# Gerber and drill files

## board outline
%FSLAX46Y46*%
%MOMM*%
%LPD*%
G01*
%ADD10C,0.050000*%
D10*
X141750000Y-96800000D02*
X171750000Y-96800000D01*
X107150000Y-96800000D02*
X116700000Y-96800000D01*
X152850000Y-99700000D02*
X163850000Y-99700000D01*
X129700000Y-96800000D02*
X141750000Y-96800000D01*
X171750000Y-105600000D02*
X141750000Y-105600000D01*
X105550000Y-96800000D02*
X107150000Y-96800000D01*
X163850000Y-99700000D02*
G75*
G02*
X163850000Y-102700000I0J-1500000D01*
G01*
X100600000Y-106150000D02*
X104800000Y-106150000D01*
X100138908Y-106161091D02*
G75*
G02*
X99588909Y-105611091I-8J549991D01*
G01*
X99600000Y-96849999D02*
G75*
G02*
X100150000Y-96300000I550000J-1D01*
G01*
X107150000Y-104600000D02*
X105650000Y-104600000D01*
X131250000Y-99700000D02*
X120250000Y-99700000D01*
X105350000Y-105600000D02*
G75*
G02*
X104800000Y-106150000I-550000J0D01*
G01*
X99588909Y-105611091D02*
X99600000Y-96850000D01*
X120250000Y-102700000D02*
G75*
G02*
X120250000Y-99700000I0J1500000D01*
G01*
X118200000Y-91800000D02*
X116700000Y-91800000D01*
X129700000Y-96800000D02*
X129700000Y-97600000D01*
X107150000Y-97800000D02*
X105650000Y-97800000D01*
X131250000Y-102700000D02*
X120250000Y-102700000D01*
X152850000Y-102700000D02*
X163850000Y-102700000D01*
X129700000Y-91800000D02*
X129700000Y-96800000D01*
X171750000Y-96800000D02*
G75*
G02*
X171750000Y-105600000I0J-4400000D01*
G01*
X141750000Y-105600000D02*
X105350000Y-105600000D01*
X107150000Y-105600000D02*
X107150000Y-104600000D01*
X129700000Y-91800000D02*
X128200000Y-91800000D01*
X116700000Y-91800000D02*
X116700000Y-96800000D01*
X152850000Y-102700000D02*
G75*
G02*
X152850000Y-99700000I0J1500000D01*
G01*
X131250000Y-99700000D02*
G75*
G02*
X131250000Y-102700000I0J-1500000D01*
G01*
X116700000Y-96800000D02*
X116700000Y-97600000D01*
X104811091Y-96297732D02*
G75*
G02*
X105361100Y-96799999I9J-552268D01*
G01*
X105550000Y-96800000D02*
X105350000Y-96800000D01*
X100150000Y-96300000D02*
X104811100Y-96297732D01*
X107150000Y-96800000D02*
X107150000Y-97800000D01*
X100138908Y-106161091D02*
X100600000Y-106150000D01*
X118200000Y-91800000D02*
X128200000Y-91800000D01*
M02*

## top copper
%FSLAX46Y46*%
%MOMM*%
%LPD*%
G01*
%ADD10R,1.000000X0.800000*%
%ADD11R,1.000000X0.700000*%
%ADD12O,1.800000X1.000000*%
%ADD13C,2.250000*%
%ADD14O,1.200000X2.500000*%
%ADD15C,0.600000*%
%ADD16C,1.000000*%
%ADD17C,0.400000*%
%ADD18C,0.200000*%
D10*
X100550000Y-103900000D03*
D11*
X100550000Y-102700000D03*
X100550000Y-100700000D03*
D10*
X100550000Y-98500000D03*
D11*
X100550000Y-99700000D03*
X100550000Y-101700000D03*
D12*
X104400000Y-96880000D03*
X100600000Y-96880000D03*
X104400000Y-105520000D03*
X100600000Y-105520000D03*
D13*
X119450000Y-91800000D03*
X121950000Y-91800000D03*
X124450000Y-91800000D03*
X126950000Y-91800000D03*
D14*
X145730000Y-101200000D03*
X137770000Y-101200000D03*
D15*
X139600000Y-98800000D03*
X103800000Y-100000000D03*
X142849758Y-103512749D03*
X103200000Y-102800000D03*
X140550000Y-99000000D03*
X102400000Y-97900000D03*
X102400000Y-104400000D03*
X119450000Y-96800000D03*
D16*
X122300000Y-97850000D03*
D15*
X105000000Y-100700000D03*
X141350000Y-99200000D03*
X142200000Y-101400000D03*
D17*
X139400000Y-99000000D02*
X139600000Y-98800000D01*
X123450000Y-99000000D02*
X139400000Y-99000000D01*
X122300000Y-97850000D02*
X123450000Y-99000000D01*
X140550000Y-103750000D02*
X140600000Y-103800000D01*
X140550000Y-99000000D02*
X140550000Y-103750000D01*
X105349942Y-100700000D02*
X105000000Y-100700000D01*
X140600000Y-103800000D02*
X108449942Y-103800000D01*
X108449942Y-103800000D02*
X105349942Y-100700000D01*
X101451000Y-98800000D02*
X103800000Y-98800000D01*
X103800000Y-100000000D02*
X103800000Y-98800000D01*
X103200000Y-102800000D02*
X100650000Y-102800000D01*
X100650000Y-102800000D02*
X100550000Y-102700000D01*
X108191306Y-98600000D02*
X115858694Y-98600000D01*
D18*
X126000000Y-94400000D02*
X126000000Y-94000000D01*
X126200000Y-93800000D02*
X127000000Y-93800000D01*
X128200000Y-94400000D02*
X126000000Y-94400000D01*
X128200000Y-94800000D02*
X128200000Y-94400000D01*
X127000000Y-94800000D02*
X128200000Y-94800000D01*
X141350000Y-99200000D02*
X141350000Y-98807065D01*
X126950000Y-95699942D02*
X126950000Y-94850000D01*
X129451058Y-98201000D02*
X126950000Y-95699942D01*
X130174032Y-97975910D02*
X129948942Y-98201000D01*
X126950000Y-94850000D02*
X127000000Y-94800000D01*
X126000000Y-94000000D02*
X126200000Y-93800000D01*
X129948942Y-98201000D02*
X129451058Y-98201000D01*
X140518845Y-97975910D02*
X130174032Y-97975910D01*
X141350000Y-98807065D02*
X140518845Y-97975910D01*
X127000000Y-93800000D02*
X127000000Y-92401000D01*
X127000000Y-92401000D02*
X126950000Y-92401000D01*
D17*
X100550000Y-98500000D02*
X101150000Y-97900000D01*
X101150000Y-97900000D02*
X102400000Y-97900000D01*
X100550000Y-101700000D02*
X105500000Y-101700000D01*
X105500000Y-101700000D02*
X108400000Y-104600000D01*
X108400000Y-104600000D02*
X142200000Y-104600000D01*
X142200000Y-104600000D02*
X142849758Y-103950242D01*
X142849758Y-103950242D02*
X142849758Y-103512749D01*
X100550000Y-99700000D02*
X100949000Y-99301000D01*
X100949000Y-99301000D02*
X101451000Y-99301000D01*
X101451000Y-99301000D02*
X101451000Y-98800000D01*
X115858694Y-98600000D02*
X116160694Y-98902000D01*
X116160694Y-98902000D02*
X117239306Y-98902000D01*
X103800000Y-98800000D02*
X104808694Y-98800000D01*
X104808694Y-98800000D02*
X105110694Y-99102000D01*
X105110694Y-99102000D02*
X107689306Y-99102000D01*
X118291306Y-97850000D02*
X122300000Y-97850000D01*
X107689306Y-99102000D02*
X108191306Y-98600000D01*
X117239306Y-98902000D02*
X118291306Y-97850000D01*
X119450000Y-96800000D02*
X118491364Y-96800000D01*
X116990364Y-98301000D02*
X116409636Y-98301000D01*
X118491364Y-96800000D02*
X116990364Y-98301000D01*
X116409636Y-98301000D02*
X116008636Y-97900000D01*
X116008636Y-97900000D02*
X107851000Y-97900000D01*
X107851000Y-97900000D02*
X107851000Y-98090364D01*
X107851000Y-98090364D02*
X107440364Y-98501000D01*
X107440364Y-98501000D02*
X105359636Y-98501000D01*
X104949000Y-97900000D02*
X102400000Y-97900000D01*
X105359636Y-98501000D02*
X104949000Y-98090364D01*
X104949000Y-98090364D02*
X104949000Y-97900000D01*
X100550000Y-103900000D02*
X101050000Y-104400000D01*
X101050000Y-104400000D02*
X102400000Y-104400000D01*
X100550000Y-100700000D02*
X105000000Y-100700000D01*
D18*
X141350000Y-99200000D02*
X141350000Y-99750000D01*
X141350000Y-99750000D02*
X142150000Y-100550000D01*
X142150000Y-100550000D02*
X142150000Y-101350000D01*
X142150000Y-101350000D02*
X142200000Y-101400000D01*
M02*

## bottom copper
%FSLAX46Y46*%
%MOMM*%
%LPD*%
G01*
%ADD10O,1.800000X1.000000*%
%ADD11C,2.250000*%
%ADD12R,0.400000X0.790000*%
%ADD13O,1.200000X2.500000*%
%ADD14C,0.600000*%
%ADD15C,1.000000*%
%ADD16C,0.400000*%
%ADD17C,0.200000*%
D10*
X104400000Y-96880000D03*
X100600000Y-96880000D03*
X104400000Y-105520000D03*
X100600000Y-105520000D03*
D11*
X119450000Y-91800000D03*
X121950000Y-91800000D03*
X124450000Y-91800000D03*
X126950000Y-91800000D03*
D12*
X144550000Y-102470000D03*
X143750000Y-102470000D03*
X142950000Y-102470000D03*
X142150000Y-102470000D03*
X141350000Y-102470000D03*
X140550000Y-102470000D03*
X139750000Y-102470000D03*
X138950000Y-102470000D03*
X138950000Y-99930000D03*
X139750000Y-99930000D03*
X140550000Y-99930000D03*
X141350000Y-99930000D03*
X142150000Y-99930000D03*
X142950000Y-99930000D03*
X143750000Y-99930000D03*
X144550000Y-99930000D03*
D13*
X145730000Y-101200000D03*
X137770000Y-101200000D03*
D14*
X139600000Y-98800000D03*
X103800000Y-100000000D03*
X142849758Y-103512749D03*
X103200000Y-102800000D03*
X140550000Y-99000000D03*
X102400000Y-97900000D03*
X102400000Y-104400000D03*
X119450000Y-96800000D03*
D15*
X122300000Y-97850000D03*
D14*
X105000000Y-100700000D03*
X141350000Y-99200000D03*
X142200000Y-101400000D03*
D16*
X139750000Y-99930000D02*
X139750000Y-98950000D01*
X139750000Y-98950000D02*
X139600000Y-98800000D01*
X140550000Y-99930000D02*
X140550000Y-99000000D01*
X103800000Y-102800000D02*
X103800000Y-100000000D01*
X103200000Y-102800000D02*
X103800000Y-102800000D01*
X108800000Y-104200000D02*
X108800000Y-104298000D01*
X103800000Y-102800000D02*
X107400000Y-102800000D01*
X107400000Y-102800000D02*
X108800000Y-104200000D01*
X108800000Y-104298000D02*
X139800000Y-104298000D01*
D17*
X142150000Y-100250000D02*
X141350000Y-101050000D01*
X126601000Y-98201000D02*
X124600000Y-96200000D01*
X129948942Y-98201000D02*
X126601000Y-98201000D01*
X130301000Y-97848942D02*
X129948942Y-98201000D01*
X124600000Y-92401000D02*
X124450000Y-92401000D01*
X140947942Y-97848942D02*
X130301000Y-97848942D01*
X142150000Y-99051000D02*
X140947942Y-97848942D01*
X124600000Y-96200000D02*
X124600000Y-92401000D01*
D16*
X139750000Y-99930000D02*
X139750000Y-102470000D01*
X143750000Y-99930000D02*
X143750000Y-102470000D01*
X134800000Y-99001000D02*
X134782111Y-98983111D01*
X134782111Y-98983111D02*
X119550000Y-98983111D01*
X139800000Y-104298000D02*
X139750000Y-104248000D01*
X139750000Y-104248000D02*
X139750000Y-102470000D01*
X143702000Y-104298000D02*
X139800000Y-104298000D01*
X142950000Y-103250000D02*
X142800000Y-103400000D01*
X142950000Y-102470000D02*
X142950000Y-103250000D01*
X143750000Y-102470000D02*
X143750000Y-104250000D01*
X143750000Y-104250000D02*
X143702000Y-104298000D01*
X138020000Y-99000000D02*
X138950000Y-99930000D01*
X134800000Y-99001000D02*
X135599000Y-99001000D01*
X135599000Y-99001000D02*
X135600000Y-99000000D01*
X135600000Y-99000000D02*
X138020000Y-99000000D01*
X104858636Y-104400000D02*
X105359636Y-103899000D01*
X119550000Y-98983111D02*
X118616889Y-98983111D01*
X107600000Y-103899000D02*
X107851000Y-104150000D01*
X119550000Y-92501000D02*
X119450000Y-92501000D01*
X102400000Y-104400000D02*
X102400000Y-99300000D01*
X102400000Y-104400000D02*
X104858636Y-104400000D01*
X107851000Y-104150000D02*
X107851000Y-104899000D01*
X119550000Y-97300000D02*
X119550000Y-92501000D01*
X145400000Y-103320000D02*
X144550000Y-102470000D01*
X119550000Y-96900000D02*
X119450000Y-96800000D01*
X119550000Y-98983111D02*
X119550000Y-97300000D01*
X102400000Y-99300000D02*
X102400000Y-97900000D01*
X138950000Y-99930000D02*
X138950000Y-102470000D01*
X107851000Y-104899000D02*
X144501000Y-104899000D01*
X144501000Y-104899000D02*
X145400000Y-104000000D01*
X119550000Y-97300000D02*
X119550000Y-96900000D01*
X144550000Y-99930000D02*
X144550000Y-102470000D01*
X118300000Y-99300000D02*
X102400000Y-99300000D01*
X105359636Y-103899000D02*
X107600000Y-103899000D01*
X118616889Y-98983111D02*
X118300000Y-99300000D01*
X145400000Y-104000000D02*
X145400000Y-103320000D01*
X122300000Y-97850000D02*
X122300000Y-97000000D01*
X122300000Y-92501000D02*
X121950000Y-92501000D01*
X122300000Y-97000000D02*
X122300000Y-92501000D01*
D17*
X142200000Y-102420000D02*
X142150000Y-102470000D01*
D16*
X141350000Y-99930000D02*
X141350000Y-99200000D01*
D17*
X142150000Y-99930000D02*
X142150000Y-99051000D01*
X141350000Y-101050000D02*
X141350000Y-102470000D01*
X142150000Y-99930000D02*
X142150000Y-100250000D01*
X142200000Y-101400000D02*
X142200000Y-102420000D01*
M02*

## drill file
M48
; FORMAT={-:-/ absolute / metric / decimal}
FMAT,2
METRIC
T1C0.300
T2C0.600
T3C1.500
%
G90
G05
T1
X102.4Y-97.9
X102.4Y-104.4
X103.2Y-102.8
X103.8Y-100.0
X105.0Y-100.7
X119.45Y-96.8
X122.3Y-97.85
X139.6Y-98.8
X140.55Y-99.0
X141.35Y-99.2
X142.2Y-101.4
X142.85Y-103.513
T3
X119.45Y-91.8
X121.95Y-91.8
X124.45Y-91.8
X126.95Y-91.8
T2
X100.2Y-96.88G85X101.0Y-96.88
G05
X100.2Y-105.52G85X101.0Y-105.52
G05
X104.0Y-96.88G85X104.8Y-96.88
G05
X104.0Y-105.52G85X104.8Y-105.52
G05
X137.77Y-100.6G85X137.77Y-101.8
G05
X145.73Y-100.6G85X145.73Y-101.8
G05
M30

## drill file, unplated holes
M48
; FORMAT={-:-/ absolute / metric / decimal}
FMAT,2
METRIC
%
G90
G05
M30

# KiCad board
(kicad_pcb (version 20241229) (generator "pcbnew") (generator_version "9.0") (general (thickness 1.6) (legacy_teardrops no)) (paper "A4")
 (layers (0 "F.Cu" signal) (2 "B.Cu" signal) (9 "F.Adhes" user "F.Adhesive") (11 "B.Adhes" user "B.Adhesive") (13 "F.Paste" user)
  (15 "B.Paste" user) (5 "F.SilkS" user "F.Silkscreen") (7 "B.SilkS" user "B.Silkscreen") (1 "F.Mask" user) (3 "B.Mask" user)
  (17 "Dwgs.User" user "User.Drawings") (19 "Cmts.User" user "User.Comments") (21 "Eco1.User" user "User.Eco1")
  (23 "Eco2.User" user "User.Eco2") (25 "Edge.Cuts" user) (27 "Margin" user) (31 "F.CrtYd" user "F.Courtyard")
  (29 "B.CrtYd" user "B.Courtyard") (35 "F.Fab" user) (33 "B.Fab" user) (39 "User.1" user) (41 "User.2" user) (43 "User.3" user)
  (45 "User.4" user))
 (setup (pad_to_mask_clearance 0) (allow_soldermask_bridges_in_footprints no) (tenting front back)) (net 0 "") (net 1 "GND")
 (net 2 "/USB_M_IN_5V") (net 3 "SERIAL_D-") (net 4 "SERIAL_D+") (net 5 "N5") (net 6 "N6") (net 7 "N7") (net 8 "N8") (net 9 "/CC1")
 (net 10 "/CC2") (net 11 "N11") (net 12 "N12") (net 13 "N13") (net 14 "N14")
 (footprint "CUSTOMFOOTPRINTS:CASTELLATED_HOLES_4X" (layer "F.Cu") (at 123.2 91.8)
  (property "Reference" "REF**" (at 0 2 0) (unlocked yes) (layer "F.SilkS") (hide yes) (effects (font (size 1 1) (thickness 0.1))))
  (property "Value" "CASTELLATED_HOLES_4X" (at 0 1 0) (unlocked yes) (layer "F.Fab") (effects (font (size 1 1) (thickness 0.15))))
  (fp_line (start -5 0) (end 5 0) (stroke (width 0.05) (type default)) (layer "Edge.Cuts"))
  (pad "1" thru_hole circle (at -3.75 0) (size 2.25 2.25) (drill 1.5) (layers "*.Cu" "*.Mask") (remove_unused_layers no) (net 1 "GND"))
  (pad "2" thru_hole circle (at -1.25 0) (size 2.25 2.25) (drill 1.5) (layers "*.Cu" "*.Mask") (remove_unused_layers no)
   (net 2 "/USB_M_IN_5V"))
  (pad "3" thru_hole circle (at 1.25 0) (size 2.25 2.25) (drill 1.5) (layers "*.Cu" "*.Mask") (remove_unused_layers no) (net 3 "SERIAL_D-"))
  (pad "4" thru_hole circle (at 3.75 0) (size 2.25 2.25) (drill 1.5) (layers "*.Cu" "*.Mask") (remove_unused_layers no) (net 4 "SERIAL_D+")))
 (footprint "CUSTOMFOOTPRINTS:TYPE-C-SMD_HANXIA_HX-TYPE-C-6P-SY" (layer "F.Cu") (at 102.475 101.2 90)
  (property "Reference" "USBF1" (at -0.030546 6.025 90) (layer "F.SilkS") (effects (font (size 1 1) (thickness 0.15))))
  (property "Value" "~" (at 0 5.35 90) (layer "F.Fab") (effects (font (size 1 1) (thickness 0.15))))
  (pad "7" thru_hole oval (at -4.32 -1.875 90) (size 1 1.8) (drill oval 0.6 1.4) (layers "*.Cu" "*.Mask") (remove_unused_layers no)
   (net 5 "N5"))
  (pad "7" thru_hole oval (at -4.32 1.925 90) (size 1 1.8) (drill oval 0.6 1.4) (layers "*.Cu" "*.Mask") (remove_unused_layers no)
   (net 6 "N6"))
  (pad "7" thru_hole oval (at 4.32 -1.875 90) (size 1 1.8) (drill oval 0.6 1.4) (layers "*.Cu" "*.Mask") (remove_unused_layers no)
   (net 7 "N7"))
  (pad "7" thru_hole oval (at 4.32 1.925 90) (size 1 1.8) (drill oval 0.6 1.4) (layers "*.Cu" "*.Mask") (remove_unused_layers no)
   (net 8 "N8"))
  (pad "A5" smd rect (at -0.5 -1.925 90) (size 0.7 1) (layers "F.Cu" "F.Mask" "F.Paste") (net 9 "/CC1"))
  (pad "A9" smd rect (at 1.5 -1.925 90) (size 0.7 1) (layers "F.Cu" "F.Mask" "F.Paste") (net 2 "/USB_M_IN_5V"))
  (pad "A12" smd rect (at 2.7 -1.925 90) (size 0.8 1) (layers "F.Cu" "F.Mask" "F.Paste") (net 1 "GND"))
  (pad "B5" smd rect (at 0.5 -1.925 90) (size 0.7 1) (layers "F.Cu" "F.Mask" "F.Paste") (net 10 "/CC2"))
  (pad "B9" smd rect (at -1.5 -1.925 90) (size 0.7 1) (layers "F.Cu" "F.Mask" "F.Paste") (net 2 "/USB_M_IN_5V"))
  (pad "B12" smd rect (at -2.7 -1.925 90) (size 0.8 1) (layers "F.Cu" "F.Mask" "F.Paste") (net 1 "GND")))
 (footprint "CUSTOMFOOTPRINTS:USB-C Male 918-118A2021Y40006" (layer "B.Cu") (at 141.75 101.2)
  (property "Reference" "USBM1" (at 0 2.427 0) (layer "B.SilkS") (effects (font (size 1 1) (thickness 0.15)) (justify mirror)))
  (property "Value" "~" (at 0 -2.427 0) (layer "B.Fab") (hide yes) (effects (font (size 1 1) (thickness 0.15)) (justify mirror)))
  (pad "1" smd rect (at 2.8 1.27) (size 0.4 0.79) (layers "B.Cu" "B.Mask" "B.Paste") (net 1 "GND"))
  (pad "2" smd rect (at 2 1.27) (size 0.4 0.79) (layers "B.Cu" "B.Mask" "B.Paste") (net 2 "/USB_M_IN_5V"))
  (pad "3" smd rect (at 1.2 1.27) (size 0.4 0.79) (layers "B.Cu" "B.Mask" "B.Paste") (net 9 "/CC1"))
  (pad "4" smd rect (at 0.4 1.27) (size 0.4 0.79) (layers "B.Cu" "B.Mask" "B.Paste") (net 4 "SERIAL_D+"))
  (pad "5" smd rect (at -0.4 1.27) (size 0.4 0.79) (layers "B.Cu" "B.Mask" "B.Paste") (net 3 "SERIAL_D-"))
  (pad "6" smd rect (at -1.2 1.27) (size 0.4 0.79) (layers "B.Cu" "B.Mask" "B.Paste") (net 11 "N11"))
  (pad "7" smd rect (at -2 1.27) (size 0.4 0.79) (layers "B.Cu" "B.Mask" "B.Paste") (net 2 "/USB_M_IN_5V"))
  (pad "8" smd rect (at -2.8 1.27) (size 0.4 0.79) (layers "B.Cu" "B.Mask" "B.Paste") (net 1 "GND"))
  (pad "9" smd rect (at -2.8 -1.27) (size 0.4 0.79) (layers "B.Cu" "B.Mask" "B.Paste") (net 1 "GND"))
  (pad "10" smd rect (at -2 -1.27) (size 0.4 0.79) (layers "B.Cu" "B.Mask" "B.Paste") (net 2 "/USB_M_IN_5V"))
  (pad "11" smd rect (at -1.2 -1.27) (size 0.4 0.79) (layers "B.Cu" "B.Mask" "B.Paste") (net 10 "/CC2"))
  (pad "12" smd rect (at -0.4 -1.27) (size 0.4 0.79) (layers "B.Cu" "B.Mask" "B.Paste") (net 4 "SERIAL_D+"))
  (pad "13" smd rect (at 0.4 -1.27) (size 0.4 0.79) (layers "B.Cu" "B.Mask" "B.Paste") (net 3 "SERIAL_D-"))
  (pad "14" smd rect (at 1.2 -1.27) (size 0.4 0.79) (layers "B.Cu" "B.Mask" "B.Paste") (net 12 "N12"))
  (pad "15" smd rect (at 2 -1.27) (size 0.4 0.79) (layers "B.Cu" "B.Mask" "B.Paste") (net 2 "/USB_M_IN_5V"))
  (pad "16" smd rect (at 2.8 -1.27) (size 0.4 0.79) (layers "B.Cu" "B.Mask" "B.Paste") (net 1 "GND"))
  (pad "17" thru_hole oval (at 3.98 0) (size 1.2 2.5) (drill oval 0.6 1.8) (layers "*.Cu" "*.Mask") (remove_unused_layers no) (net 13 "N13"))
  (pad "18" thru_hole oval (at -3.98 0) (size 1.2 2.5) (drill oval 0.6 1.8) (layers "*.Cu" "*.Mask") (remove_unused_layers no)
   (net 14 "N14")))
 (gr_line (start 141.75 96.8) (end 171.75 96.8) (stroke (width 0.05) (type solid)) (layer "Edge.Cuts"))
 (gr_line (start 107.15 96.8) (end 116.7 96.8) (stroke (width 0.05) (type default)) (layer "Edge.Cuts"))
 (gr_line (start 152.85 99.7) (end 163.85 99.7) (stroke (width 0.05) (type default)) (layer "Edge.Cuts"))
 (gr_line (start 129.7 96.8) (end 141.75 96.8) (stroke (width 0.05) (type default)) (layer "Edge.Cuts"))
 (gr_line (start 171.75 105.6) (end 141.75 105.6) (stroke (width 0.05) (type default)) (layer "Edge.Cuts"))
 (gr_line (start 105.55 96.8) (end 107.15 96.8) (stroke (width 0.05) (type default)) (layer "Edge.Cuts"))
 (gr_arc (start 163.85 99.7) (mid 165.35 101.2) (end 163.85 102.7) (stroke (width 0.05) (type default)) (layer "Edge.Cuts"))
 (gr_line (start 100.6 106.15) (end 104.8 106.15) (stroke (width 0.05) (type default)) (layer "Edge.Cuts"))
 (gr_arc (start 100.138908 106.161091) (mid 99.749997 106.000002) (end 99.588909 105.611091) (stroke (width 0.05) (type default))
  (layer "Edge.Cuts"))
 (gr_arc (start 99.6 96.849999) (mid 99.761092 96.461091) (end 100.15 96.3) (stroke (width 0.05) (type default)) (layer "Edge.Cuts"))
 (gr_line (start 107.15 104.6) (end 105.65 104.6) (stroke (width 0.05) (type default)) (layer "Edge.Cuts"))
 (gr_line (start 131.25 99.7) (end 120.25 99.7) (stroke (width 0.05) (type default)) (layer "Edge.Cuts"))
 (gr_arc (start 105.35 105.6) (mid 105.188909 105.988909) (end 104.8 106.15) (stroke (width 0.05) (type default)) (layer "Edge.Cuts"))
 (gr_line (start 99.588909 105.611091) (end 99.6 96.85) (stroke (width 0.05) (type default)) (layer "Edge.Cuts"))
 (gr_arc (start 120.25 102.7) (mid 118.75 101.2) (end 120.25 99.7) (stroke (width 0.05) (type default)) (layer "Edge.Cuts"))
 (gr_line (start 118.2 91.8) (end 116.7 91.8) (stroke (width 0.05) (type default)) (layer "Edge.Cuts"))
 (gr_line (start 129.7 96.8) (end 129.7 97.6) (stroke (width 0.05) (type default)) (layer "Edge.Cuts"))
 (gr_line (start 107.15 97.8) (end 105.65 97.8) (stroke (width 0.05) (type default)) (layer "Edge.Cuts"))
 (gr_line (start 131.25 102.7) (end 120.25 102.7) (stroke (width 0.05) (type default)) (layer "Edge.Cuts"))
 (gr_line (start 152.85 102.7) (end 163.85 102.7) (stroke (width 0.05) (type default)) (layer "Edge.Cuts"))
 (gr_line (start 129.7 91.8) (end 129.7 96.8) (stroke (width 0.05) (type default)) (layer "Edge.Cuts"))
 (gr_arc (start 171.75 96.8) (mid 176.15 101.2) (end 171.75 105.6) (stroke (width 0.05) (type default)) (layer "Edge.Cuts"))
 (gr_line (start 141.75 105.6) (end 105.35 105.6) (stroke (width 0.05) (type default)) (layer "Edge.Cuts"))
 (gr_line (start 107.15 105.6) (end 107.15 104.6) (stroke (width 0.05) (type default)) (layer "Edge.Cuts"))
 (gr_line (start 129.7 91.8) (end 128.2 91.8) (stroke (width 0.05) (type default)) (layer "Edge.Cuts"))
 (gr_line (start 116.7 91.8) (end 116.7 96.8) (stroke (width 0.05) (type default)) (layer "Edge.Cuts"))
 (gr_arc (start 152.85 102.7) (mid 151.35 101.2) (end 152.85 99.7) (stroke (width 0.05) (type default)) (layer "Edge.Cuts"))
 (gr_arc (start 131.25 99.7) (mid 132.75 101.2) (end 131.25 102.7) (stroke (width 0.05) (type default)) (layer "Edge.Cuts"))
 (gr_line (start 116.7 96.8) (end 116.7 97.6) (stroke (width 0.05) (type default)) (layer "Edge.Cuts"))
 (gr_arc (start 104.811091 96.297732) (mid 105.183512 96.44219) (end 105.361091 96.8) (stroke (width 0.05) (type default))
  (layer "Edge.Cuts"))
 (gr_line (start 105.55 96.8) (end 105.35 96.8) (stroke (width 0.05) (type default)) (layer "Edge.Cuts"))
 (gr_line (start 100.15 96.3) (end 104.8111 96.297732) (stroke (width 0.05) (type default)) (layer "Edge.Cuts"))
 (gr_line (start 107.15 96.8) (end 107.15 97.8) (stroke (width 0.05) (type default)) (layer "Edge.Cuts"))
 (gr_line (start 100.138908 106.161091) (end 100.6 106.15) (stroke (width 0.05) (type default)) (layer "Edge.Cuts"))
 (segment (start 104.949 97.9) (end 102.4 97.9) (width 0.4) (layer "F.Cu") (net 1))
 (segment (start 119.45 96.8) (end 118.491364 96.8) (width 0.4) (layer "F.Cu") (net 1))
 (segment (start 107.851 98.090364) (end 107.440364 98.501) (width 0.4) (layer "F.Cu") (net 1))
 (segment (start 107.440364 98.501) (end 105.359636 98.501) (width 0.4) (layer "F.Cu") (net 1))
 (segment (start 116.990364 98.301) (end 116.409636 98.301) (width 0.4) (layer "F.Cu") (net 1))
 (segment (start 101.15 97.9) (end 102.4 97.9) (width 0.4) (layer "F.Cu") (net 1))
 (segment (start 100.55 103.9) (end 101.05 104.4) (width 0.4) (layer "F.Cu") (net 1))
 (segment (start 104.949 98.090364) (end 104.949 97.9) (width 0.4) (layer "F.Cu") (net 1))
 (segment (start 101.05 104.4) (end 102.4 104.4) (width 0.4) (layer "F.Cu") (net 1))
 (segment (start 105.359636 98.501) (end 104.949 98.090364) (width 0.4) (layer "F.Cu") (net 1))
 (segment (start 116.409636 98.301) (end 116.008636 97.9) (width 0.4) (layer "F.Cu") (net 1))
 (segment (start 107.851 97.9) (end 107.851 98.090364) (width 0.4) (layer "F.Cu") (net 1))
 (segment (start 118.491364 96.8) (end 116.990364 98.301) (width 0.4) (layer "F.Cu") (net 1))
 (segment (start 116.008636 97.9) (end 107.851 97.9) (width 0.4) (layer "F.Cu") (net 1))
 (segment (start 100.55 98.5) (end 101.15 97.9) (width 0.4) (layer "F.Cu") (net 1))
 (via (at 102.4 97.9) (size 0.6) (drill 0.3) (layers "F.Cu" "B.Cu") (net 1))
 (via (at 102.4 104.4) (size 0.6) (drill 0.3) (layers "F.Cu" "B.Cu") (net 1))
 (via (at 119.45 96.8) (size 0.6) (drill 0.3) (layers "F.Cu" "B.Cu") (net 1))
 (segment (start 104.858636 104.4) (end 105.359636 103.899) (width 0.4) (layer "B.Cu") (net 1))
 (segment (start 119.55 98.983111) (end 118.616889 98.983111) (width 0.4) (layer "B.Cu") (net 1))
 (segment (start 107.6 103.899) (end 107.851 104.15) (width 0.4) (layer "B.Cu") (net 1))
 (segment (start 119.55 92.501) (end 119.45 92.501) (width 0.4) (layer "B.Cu") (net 1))
 (segment (start 138.02 99) (end 138.95 99.93) (width 0.4) (layer "B.Cu") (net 1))
 (segment (start 134.8 99.001) (end 134.782111 98.983111) (width 0.4) (layer "B.Cu") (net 1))
 (segment (start 102.4 104.4) (end 102.4 99.3) (width 0.4) (layer "B.Cu") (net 1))
 (segment (start 102.4 104.4) (end 104.858636 104.4) (width 0.4) (layer "B.Cu") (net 1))
 (segment (start 107.851 104.15) (end 107.851 104.899) (width 0.4) (layer "B.Cu") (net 1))
 (segment (start 134.8 99.001) (end 135.599 99.001) (width 0.4) (layer "B.Cu") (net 1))
 (segment (start 135.599 99.001) (end 135.6 99) (width 0.4) (layer "B.Cu") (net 1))
 (segment (start 119.55 97.3) (end 119.55 92.501) (width 0.4) (layer "B.Cu") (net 1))
 (segment (start 145.4 103.32) (end 144.55 102.47) (width 0.4) (layer "B.Cu") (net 1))
 (segment (start 119.55 96.9) (end 119.45 96.8) (width 0.4) (layer "B.Cu") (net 1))
 (segment (start 119.55 98.983111) (end 119.55 97.3) (width 0.4) (layer "B.Cu") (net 1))
 (segment (start 102.4 99.3) (end 102.4 97.9) (width 0.4) (layer "B.Cu") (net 1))
 (segment (start 138.95 99.93) (end 138.95 102.47) (width 0.4) (layer "B.Cu") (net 1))
 (segment (start 107.851 104.899) (end 144.501 104.899) (width 0.4) (layer "B.Cu") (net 1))
 (segment (start 144.501 104.899) (end 145.4 104) (width 0.4) (layer "B.Cu") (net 1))
 (segment (start 119.55 97.3) (end 119.55 96.9) (width 0.4) (layer "B.Cu") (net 1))
 (segment (start 144.55 99.93) (end 144.55 102.47) (width 0.4) (layer "B.Cu") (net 1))
 (segment (start 118.3 99.3) (end 102.4 99.3) (width 0.4) (layer "B.Cu") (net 1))
 (segment (start 134.782111 98.983111) (end 119.55 98.983111) (width 0.4) (layer "B.Cu") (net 1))
 (segment (start 105.359636 103.899) (end 107.6 103.899) (width 0.4) (layer "B.Cu") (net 1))
 (segment (start 135.6 99) (end 138.02 99) (width 0.4) (layer "B.Cu") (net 1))
 (segment (start 118.616889 98.983111) (end 118.3 99.3) (width 0.4) (layer "B.Cu") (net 1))
 (segment (start 145.4 104) (end 145.4 103.32) (width 0.4) (layer "B.Cu") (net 1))
 (segment (start 103.8 98.8) (end 104.808694 98.8) (width 0.4) (layer "F.Cu") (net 2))
 (segment (start 103.8 100) (end 103.8 98.8) (width 0.4) (layer "F.Cu") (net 2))
 (segment (start 108.191306 98.6) (end 115.858694 98.6) (width 0.4) (layer "F.Cu") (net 2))
 (segment (start 139.4 99) (end 139.6 98.8) (width 0.4) (layer "F.Cu") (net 2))
 (segment (start 105.110694 99.102) (end 107.689306 99.102) (width 0.4) (layer "F.Cu") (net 2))
 (segment (start 103.2 102.8) (end 100.65 102.8) (width 0.4) (layer "F.Cu") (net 2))
 (segment (start 100.65 102.8) (end 100.55 102.7) (width 0.4) (layer "F.Cu") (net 2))
 (segment (start 117.239306 98.902) (end 118.291306 97.85) (width 0.4) (layer "F.Cu") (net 2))
 (segment (start 123.45 99) (end 139.4 99) (width 0.4) (layer "F.Cu") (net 2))
 (segment (start 101.451 99.301) (end 101.451 98.8) (width 0.4) (layer "F.Cu") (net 2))
 (segment (start 101.451 98.8) (end 103.8 98.8) (width 0.4) (layer "F.Cu") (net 2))
 (segment (start 104.808694 98.8) (end 105.110694 99.102) (width 0.4) (layer "F.Cu") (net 2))
 (segment (start 100.949 99.301) (end 101.451 99.301) (width 0.4) (layer "F.Cu") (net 2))
 (segment (start 107.689306 99.102) (end 108.191306 98.6) (width 0.4) (layer "F.Cu") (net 2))
 (segment (start 115.858694 98.6) (end 116.160694 98.902) (width 0.4) (layer "F.Cu") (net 2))
 (segment (start 116.160694 98.902) (end 117.239306 98.902) (width 0.4) (layer "F.Cu") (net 2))
 (segment (start 122.3 97.85) (end 123.45 99) (width 0.4) (layer "F.Cu") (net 2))
 (segment (start 118.291306 97.85) (end 122.3 97.85) (width 0.4) (layer "F.Cu") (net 2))
 (segment (start 100.55 99.7) (end 100.949 99.301) (width 0.4) (layer "F.Cu") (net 2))
 (via (at 103.2 102.8) (size 0.6) (drill 0.3) (layers "F.Cu" "B.Cu") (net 2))
 (via (at 122.3 97.85) (size 1) (drill 0.3) (layers "F.Cu" "B.Cu") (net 2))
 (via (at 139.6 98.8) (size 0.6) (drill 0.3) (layers "F.Cu" "B.Cu") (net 2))
 (via (at 103.8 100) (size 0.6) (drill 0.3) (layers "F.Cu" "B.Cu") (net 2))
 (segment (start 139.75 99.93) (end 139.75 102.47) (width 0.4) (layer "B.Cu") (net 2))
 (segment (start 107.4 102.8) (end 108.8 104.2) (width 0.4) (layer "B.Cu") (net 2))
 (segment (start 139.75 98.95) (end 139.6 98.8) (width 0.4) (layer "B.Cu") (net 2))
 (segment (start 103.2 102.8) (end 103.8 102.8) (width 0.4) (layer "B.Cu") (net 2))
 (segment (start 103.8 102.8) (end 103.8 100) (width 0.4) (layer "B.Cu") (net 2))
 (segment (start 103.8 102.8) (end 107.4 102.8) (width 0.4) (layer "B.Cu") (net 2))
 (segment (start 122.3 97.85) (end 122.3 97) (width 0.4) (layer "B.Cu") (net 2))
 (segment (start 108.8 104.298) (end 139.8 104.298) (width 0.4) (layer "B.Cu") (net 2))
 (segment (start 143.702 104.298) (end 139.8 104.298) (width 0.4) (layer "B.Cu") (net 2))
 (segment (start 143.75 99.93) (end 143.75 102.47) (width 0.4) (layer "B.Cu") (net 2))
 (segment (start 143.75 104.25) (end 143.702 104.298) (width 0.4) (layer "B.Cu") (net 2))
 (segment (start 122.3 92.501) (end 121.95 92.501) (width 0.4) (layer "B.Cu") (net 2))
 (segment (start 139.8 104.298) (end 139.75 104.248) (width 0.4) (layer "B.Cu") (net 2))
 (segment (start 143.75 102.47) (end 143.75 104.25) (width 0.4) (layer "B.Cu") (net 2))
 (segment (start 139.75 104.248) (end 139.75 102.47) (width 0.4) (layer "B.Cu") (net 2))
 (segment (start 139.75 99.93) (end 139.75 98.95) (width 0.4) (layer "B.Cu") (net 2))
 (segment (start 122.3 97) (end 122.3 92.501) (width 0.4) (layer "B.Cu") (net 2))
 (segment (start 108.8 104.2) (end 108.8 104.298) (width 0.4) (layer "B.Cu") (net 2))
 (segment (start 140.6 103.8) (end 108.449942 103.8) (width 0.4) (layer "F.Cu") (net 10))
 (segment (start 140.55 103.75) (end 140.6 103.8) (width 0.4) (layer "F.Cu") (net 10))
 (segment (start 105.349942 100.7) (end 105 100.7) (width 0.4) (layer "F.Cu") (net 10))
 (segment (start 108.449942 103.8) (end 105.349942 100.7) (width 0.4) (layer "F.Cu") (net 10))
 (segment (start 140.55 99) (end 140.55 103.75) (width 0.4) (layer "F.Cu") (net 10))
 (segment (start 100.55 100.7) (end 105 100.7) (width 0.4) (layer "F.Cu") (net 10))
 (via (at 140.55 99) (size 0.6) (drill 0.3) (layers "F.Cu" "B.Cu") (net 10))
 (via (at 105 100.7) (size 0.6) (drill 0.3) (layers "F.Cu" "B.Cu") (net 10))
 (segment (start 140.55 99.93) (end 140.55 99) (width 0.4) (layer "B.Cu") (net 10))
 (segment (start 108.4 104.6) (end 142.2 104.6) (width 0.4) (layer "F.Cu") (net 9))
 (segment (start 142.849758 103.950242) (end 142.849758 103.512749) (width 0.4) (layer "F.Cu") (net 9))
 (segment (start 142.2 104.6) (end 142.849758 103.950242) (width 0.4) (layer "F.Cu") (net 9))
 (segment (start 105.5 101.7) (end 108.4 104.6) (width 0.4) (layer "F.Cu") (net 9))
 (segment (start 100.55 101.7) (end 105.5 101.7) (width 0.4) (layer "F.Cu") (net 9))
 (via (at 142.849758 103.512749) (size 0.6) (drill 0.3) (layers "F.Cu" "B.Cu") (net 9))
 (segment (start 142.95 102.47) (end 142.95 103.25) (width 0.4) (layer "B.Cu") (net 9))
 (segment (start 142.95 103.25) (end 142.8 103.4) (width 0.4) (layer "B.Cu") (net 9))
 (segment (start 126 94) (end 126.2 93.8) (width 0.2) (layer "F.Cu") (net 4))
 (segment (start 126.2 93.8) (end 127 93.8) (width 0.2) (layer "F.Cu") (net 4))
 (segment (start 141.35 98.807065) (end 140.518845 97.97591) (width 0.2) (layer "F.Cu") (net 4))
 (segment (start 127 92.401) (end 126.95 92.401) (width 0.2) (layer "F.Cu") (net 4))
 (segment (start 128.2 94.4) (end 126 94.4) (width 0.2) (layer "F.Cu") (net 4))
 (segment (start 141.35 99.2) (end 141.35 99.75) (width 0.2) (layer "F.Cu") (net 4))
 (segment (start 127 93.8) (end 127 92.401) (width 0.2) (layer "F.Cu") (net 4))
 (segment (start 141.35 99.75) (end 142.15 100.55) (width 0.2) (layer "F.Cu") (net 4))
 (segment (start 126.95 94.85) (end 127 94.8) (width 0.2) (layer "F.Cu") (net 4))
 (segment (start 126.95 95.699942) (end 126.95 94.85) (width 0.2) (layer "F.Cu") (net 4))
 (segment (start 130.174032 97.97591) (end 129.948942 98.201) (width 0.2) (layer "F.Cu") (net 4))
 (segment (start 128.2 94.8) (end 128.2 94.4) (width 0.2) (layer "F.Cu") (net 4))
 (segment (start 129.948942 98.201) (end 129.451058 98.201) (width 0.2) (layer "F.Cu") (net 4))
 (segment (start 126 94.4) (end 126 94) (width 0.2) (layer "F.Cu") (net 4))
 (segment (start 129.451058 98.201) (end 126.95 95.699942) (width 0.2) (layer "F.Cu") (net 4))
 (segment (start 140.518845 97.97591) (end 130.174032 97.97591) (width 0.2) (layer "F.Cu") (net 4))
 (segment (start 142.15 100.55) (end 142.15 101.35) (width 0.2) (layer "F.Cu") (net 4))
 (segment (start 141.35 99.2) (end 141.35 98.807065) (width 0.2) (layer "F.Cu") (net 4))
 (segment (start 142.15 101.35) (end 142.2 101.4) (width 0.2) (layer "F.Cu") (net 4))
 (segment (start 127 94.8) (end 128.2 94.8) (width 0.2) (layer "F.Cu") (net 4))
 (via (at 141.35 99.2) (size 0.6) (drill 0.3) (layers "F.Cu" "B.Cu") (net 4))
 (via (at 142.2 101.4) (size 0.6) (drill 0.3) (layers "F.Cu" "B.Cu") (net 4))
 (segment (start 142.2 102.42) (end 142.15 102.47) (width 0.2) (layer "B.Cu") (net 4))
 (segment (start 142.2 101.4) (end 142.2 102.42) (width 0.2) (layer "B.Cu") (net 4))
 (segment (start 141.35 99.93) (end 141.35 99.2) (width 0.4) (layer "B.Cu") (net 4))
 (segment (start 124.6 96.2) (end 124.6 92.401) (width 0.2) (layer "B.Cu") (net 3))
 (segment (start 126.601 98.201) (end 124.6 96.2) (width 0.2) (layer "B.Cu") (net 3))
 (segment (start 124.6 92.401) (end 124.45 92.401) (width 0.2) (layer "B.Cu") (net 3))
 (segment (start 142.15 99.93) (end 142.15 99.051) (width 0.2) (layer "B.Cu") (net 3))
 (segment (start 129.948942 98.201) (end 126.601 98.201) (width 0.2) (layer "B.Cu") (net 3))
 (segment (start 142.15 100.25) (end 141.35 101.05) (width 0.2) (layer "B.Cu") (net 3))
 (segment (start 140.947942 97.848942) (end 130.301 97.848942) (width 0.2) (layer "B.Cu") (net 3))
 (segment (start 141.35 101.05) (end 141.35 102.47) (width 0.2) (layer "B.Cu") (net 3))
 (segment (start 142.15 99.93) (end 142.15 100.25) (width 0.2) (layer "B.Cu") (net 3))
 (segment (start 130.301 97.848942) (end 129.948942 98.201) (width 0.2) (layer "B.Cu") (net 3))
 (segment (start 142.15 99.051) (end 140.947942 97.848942) (width 0.2) (layer "B.Cu") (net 3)))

